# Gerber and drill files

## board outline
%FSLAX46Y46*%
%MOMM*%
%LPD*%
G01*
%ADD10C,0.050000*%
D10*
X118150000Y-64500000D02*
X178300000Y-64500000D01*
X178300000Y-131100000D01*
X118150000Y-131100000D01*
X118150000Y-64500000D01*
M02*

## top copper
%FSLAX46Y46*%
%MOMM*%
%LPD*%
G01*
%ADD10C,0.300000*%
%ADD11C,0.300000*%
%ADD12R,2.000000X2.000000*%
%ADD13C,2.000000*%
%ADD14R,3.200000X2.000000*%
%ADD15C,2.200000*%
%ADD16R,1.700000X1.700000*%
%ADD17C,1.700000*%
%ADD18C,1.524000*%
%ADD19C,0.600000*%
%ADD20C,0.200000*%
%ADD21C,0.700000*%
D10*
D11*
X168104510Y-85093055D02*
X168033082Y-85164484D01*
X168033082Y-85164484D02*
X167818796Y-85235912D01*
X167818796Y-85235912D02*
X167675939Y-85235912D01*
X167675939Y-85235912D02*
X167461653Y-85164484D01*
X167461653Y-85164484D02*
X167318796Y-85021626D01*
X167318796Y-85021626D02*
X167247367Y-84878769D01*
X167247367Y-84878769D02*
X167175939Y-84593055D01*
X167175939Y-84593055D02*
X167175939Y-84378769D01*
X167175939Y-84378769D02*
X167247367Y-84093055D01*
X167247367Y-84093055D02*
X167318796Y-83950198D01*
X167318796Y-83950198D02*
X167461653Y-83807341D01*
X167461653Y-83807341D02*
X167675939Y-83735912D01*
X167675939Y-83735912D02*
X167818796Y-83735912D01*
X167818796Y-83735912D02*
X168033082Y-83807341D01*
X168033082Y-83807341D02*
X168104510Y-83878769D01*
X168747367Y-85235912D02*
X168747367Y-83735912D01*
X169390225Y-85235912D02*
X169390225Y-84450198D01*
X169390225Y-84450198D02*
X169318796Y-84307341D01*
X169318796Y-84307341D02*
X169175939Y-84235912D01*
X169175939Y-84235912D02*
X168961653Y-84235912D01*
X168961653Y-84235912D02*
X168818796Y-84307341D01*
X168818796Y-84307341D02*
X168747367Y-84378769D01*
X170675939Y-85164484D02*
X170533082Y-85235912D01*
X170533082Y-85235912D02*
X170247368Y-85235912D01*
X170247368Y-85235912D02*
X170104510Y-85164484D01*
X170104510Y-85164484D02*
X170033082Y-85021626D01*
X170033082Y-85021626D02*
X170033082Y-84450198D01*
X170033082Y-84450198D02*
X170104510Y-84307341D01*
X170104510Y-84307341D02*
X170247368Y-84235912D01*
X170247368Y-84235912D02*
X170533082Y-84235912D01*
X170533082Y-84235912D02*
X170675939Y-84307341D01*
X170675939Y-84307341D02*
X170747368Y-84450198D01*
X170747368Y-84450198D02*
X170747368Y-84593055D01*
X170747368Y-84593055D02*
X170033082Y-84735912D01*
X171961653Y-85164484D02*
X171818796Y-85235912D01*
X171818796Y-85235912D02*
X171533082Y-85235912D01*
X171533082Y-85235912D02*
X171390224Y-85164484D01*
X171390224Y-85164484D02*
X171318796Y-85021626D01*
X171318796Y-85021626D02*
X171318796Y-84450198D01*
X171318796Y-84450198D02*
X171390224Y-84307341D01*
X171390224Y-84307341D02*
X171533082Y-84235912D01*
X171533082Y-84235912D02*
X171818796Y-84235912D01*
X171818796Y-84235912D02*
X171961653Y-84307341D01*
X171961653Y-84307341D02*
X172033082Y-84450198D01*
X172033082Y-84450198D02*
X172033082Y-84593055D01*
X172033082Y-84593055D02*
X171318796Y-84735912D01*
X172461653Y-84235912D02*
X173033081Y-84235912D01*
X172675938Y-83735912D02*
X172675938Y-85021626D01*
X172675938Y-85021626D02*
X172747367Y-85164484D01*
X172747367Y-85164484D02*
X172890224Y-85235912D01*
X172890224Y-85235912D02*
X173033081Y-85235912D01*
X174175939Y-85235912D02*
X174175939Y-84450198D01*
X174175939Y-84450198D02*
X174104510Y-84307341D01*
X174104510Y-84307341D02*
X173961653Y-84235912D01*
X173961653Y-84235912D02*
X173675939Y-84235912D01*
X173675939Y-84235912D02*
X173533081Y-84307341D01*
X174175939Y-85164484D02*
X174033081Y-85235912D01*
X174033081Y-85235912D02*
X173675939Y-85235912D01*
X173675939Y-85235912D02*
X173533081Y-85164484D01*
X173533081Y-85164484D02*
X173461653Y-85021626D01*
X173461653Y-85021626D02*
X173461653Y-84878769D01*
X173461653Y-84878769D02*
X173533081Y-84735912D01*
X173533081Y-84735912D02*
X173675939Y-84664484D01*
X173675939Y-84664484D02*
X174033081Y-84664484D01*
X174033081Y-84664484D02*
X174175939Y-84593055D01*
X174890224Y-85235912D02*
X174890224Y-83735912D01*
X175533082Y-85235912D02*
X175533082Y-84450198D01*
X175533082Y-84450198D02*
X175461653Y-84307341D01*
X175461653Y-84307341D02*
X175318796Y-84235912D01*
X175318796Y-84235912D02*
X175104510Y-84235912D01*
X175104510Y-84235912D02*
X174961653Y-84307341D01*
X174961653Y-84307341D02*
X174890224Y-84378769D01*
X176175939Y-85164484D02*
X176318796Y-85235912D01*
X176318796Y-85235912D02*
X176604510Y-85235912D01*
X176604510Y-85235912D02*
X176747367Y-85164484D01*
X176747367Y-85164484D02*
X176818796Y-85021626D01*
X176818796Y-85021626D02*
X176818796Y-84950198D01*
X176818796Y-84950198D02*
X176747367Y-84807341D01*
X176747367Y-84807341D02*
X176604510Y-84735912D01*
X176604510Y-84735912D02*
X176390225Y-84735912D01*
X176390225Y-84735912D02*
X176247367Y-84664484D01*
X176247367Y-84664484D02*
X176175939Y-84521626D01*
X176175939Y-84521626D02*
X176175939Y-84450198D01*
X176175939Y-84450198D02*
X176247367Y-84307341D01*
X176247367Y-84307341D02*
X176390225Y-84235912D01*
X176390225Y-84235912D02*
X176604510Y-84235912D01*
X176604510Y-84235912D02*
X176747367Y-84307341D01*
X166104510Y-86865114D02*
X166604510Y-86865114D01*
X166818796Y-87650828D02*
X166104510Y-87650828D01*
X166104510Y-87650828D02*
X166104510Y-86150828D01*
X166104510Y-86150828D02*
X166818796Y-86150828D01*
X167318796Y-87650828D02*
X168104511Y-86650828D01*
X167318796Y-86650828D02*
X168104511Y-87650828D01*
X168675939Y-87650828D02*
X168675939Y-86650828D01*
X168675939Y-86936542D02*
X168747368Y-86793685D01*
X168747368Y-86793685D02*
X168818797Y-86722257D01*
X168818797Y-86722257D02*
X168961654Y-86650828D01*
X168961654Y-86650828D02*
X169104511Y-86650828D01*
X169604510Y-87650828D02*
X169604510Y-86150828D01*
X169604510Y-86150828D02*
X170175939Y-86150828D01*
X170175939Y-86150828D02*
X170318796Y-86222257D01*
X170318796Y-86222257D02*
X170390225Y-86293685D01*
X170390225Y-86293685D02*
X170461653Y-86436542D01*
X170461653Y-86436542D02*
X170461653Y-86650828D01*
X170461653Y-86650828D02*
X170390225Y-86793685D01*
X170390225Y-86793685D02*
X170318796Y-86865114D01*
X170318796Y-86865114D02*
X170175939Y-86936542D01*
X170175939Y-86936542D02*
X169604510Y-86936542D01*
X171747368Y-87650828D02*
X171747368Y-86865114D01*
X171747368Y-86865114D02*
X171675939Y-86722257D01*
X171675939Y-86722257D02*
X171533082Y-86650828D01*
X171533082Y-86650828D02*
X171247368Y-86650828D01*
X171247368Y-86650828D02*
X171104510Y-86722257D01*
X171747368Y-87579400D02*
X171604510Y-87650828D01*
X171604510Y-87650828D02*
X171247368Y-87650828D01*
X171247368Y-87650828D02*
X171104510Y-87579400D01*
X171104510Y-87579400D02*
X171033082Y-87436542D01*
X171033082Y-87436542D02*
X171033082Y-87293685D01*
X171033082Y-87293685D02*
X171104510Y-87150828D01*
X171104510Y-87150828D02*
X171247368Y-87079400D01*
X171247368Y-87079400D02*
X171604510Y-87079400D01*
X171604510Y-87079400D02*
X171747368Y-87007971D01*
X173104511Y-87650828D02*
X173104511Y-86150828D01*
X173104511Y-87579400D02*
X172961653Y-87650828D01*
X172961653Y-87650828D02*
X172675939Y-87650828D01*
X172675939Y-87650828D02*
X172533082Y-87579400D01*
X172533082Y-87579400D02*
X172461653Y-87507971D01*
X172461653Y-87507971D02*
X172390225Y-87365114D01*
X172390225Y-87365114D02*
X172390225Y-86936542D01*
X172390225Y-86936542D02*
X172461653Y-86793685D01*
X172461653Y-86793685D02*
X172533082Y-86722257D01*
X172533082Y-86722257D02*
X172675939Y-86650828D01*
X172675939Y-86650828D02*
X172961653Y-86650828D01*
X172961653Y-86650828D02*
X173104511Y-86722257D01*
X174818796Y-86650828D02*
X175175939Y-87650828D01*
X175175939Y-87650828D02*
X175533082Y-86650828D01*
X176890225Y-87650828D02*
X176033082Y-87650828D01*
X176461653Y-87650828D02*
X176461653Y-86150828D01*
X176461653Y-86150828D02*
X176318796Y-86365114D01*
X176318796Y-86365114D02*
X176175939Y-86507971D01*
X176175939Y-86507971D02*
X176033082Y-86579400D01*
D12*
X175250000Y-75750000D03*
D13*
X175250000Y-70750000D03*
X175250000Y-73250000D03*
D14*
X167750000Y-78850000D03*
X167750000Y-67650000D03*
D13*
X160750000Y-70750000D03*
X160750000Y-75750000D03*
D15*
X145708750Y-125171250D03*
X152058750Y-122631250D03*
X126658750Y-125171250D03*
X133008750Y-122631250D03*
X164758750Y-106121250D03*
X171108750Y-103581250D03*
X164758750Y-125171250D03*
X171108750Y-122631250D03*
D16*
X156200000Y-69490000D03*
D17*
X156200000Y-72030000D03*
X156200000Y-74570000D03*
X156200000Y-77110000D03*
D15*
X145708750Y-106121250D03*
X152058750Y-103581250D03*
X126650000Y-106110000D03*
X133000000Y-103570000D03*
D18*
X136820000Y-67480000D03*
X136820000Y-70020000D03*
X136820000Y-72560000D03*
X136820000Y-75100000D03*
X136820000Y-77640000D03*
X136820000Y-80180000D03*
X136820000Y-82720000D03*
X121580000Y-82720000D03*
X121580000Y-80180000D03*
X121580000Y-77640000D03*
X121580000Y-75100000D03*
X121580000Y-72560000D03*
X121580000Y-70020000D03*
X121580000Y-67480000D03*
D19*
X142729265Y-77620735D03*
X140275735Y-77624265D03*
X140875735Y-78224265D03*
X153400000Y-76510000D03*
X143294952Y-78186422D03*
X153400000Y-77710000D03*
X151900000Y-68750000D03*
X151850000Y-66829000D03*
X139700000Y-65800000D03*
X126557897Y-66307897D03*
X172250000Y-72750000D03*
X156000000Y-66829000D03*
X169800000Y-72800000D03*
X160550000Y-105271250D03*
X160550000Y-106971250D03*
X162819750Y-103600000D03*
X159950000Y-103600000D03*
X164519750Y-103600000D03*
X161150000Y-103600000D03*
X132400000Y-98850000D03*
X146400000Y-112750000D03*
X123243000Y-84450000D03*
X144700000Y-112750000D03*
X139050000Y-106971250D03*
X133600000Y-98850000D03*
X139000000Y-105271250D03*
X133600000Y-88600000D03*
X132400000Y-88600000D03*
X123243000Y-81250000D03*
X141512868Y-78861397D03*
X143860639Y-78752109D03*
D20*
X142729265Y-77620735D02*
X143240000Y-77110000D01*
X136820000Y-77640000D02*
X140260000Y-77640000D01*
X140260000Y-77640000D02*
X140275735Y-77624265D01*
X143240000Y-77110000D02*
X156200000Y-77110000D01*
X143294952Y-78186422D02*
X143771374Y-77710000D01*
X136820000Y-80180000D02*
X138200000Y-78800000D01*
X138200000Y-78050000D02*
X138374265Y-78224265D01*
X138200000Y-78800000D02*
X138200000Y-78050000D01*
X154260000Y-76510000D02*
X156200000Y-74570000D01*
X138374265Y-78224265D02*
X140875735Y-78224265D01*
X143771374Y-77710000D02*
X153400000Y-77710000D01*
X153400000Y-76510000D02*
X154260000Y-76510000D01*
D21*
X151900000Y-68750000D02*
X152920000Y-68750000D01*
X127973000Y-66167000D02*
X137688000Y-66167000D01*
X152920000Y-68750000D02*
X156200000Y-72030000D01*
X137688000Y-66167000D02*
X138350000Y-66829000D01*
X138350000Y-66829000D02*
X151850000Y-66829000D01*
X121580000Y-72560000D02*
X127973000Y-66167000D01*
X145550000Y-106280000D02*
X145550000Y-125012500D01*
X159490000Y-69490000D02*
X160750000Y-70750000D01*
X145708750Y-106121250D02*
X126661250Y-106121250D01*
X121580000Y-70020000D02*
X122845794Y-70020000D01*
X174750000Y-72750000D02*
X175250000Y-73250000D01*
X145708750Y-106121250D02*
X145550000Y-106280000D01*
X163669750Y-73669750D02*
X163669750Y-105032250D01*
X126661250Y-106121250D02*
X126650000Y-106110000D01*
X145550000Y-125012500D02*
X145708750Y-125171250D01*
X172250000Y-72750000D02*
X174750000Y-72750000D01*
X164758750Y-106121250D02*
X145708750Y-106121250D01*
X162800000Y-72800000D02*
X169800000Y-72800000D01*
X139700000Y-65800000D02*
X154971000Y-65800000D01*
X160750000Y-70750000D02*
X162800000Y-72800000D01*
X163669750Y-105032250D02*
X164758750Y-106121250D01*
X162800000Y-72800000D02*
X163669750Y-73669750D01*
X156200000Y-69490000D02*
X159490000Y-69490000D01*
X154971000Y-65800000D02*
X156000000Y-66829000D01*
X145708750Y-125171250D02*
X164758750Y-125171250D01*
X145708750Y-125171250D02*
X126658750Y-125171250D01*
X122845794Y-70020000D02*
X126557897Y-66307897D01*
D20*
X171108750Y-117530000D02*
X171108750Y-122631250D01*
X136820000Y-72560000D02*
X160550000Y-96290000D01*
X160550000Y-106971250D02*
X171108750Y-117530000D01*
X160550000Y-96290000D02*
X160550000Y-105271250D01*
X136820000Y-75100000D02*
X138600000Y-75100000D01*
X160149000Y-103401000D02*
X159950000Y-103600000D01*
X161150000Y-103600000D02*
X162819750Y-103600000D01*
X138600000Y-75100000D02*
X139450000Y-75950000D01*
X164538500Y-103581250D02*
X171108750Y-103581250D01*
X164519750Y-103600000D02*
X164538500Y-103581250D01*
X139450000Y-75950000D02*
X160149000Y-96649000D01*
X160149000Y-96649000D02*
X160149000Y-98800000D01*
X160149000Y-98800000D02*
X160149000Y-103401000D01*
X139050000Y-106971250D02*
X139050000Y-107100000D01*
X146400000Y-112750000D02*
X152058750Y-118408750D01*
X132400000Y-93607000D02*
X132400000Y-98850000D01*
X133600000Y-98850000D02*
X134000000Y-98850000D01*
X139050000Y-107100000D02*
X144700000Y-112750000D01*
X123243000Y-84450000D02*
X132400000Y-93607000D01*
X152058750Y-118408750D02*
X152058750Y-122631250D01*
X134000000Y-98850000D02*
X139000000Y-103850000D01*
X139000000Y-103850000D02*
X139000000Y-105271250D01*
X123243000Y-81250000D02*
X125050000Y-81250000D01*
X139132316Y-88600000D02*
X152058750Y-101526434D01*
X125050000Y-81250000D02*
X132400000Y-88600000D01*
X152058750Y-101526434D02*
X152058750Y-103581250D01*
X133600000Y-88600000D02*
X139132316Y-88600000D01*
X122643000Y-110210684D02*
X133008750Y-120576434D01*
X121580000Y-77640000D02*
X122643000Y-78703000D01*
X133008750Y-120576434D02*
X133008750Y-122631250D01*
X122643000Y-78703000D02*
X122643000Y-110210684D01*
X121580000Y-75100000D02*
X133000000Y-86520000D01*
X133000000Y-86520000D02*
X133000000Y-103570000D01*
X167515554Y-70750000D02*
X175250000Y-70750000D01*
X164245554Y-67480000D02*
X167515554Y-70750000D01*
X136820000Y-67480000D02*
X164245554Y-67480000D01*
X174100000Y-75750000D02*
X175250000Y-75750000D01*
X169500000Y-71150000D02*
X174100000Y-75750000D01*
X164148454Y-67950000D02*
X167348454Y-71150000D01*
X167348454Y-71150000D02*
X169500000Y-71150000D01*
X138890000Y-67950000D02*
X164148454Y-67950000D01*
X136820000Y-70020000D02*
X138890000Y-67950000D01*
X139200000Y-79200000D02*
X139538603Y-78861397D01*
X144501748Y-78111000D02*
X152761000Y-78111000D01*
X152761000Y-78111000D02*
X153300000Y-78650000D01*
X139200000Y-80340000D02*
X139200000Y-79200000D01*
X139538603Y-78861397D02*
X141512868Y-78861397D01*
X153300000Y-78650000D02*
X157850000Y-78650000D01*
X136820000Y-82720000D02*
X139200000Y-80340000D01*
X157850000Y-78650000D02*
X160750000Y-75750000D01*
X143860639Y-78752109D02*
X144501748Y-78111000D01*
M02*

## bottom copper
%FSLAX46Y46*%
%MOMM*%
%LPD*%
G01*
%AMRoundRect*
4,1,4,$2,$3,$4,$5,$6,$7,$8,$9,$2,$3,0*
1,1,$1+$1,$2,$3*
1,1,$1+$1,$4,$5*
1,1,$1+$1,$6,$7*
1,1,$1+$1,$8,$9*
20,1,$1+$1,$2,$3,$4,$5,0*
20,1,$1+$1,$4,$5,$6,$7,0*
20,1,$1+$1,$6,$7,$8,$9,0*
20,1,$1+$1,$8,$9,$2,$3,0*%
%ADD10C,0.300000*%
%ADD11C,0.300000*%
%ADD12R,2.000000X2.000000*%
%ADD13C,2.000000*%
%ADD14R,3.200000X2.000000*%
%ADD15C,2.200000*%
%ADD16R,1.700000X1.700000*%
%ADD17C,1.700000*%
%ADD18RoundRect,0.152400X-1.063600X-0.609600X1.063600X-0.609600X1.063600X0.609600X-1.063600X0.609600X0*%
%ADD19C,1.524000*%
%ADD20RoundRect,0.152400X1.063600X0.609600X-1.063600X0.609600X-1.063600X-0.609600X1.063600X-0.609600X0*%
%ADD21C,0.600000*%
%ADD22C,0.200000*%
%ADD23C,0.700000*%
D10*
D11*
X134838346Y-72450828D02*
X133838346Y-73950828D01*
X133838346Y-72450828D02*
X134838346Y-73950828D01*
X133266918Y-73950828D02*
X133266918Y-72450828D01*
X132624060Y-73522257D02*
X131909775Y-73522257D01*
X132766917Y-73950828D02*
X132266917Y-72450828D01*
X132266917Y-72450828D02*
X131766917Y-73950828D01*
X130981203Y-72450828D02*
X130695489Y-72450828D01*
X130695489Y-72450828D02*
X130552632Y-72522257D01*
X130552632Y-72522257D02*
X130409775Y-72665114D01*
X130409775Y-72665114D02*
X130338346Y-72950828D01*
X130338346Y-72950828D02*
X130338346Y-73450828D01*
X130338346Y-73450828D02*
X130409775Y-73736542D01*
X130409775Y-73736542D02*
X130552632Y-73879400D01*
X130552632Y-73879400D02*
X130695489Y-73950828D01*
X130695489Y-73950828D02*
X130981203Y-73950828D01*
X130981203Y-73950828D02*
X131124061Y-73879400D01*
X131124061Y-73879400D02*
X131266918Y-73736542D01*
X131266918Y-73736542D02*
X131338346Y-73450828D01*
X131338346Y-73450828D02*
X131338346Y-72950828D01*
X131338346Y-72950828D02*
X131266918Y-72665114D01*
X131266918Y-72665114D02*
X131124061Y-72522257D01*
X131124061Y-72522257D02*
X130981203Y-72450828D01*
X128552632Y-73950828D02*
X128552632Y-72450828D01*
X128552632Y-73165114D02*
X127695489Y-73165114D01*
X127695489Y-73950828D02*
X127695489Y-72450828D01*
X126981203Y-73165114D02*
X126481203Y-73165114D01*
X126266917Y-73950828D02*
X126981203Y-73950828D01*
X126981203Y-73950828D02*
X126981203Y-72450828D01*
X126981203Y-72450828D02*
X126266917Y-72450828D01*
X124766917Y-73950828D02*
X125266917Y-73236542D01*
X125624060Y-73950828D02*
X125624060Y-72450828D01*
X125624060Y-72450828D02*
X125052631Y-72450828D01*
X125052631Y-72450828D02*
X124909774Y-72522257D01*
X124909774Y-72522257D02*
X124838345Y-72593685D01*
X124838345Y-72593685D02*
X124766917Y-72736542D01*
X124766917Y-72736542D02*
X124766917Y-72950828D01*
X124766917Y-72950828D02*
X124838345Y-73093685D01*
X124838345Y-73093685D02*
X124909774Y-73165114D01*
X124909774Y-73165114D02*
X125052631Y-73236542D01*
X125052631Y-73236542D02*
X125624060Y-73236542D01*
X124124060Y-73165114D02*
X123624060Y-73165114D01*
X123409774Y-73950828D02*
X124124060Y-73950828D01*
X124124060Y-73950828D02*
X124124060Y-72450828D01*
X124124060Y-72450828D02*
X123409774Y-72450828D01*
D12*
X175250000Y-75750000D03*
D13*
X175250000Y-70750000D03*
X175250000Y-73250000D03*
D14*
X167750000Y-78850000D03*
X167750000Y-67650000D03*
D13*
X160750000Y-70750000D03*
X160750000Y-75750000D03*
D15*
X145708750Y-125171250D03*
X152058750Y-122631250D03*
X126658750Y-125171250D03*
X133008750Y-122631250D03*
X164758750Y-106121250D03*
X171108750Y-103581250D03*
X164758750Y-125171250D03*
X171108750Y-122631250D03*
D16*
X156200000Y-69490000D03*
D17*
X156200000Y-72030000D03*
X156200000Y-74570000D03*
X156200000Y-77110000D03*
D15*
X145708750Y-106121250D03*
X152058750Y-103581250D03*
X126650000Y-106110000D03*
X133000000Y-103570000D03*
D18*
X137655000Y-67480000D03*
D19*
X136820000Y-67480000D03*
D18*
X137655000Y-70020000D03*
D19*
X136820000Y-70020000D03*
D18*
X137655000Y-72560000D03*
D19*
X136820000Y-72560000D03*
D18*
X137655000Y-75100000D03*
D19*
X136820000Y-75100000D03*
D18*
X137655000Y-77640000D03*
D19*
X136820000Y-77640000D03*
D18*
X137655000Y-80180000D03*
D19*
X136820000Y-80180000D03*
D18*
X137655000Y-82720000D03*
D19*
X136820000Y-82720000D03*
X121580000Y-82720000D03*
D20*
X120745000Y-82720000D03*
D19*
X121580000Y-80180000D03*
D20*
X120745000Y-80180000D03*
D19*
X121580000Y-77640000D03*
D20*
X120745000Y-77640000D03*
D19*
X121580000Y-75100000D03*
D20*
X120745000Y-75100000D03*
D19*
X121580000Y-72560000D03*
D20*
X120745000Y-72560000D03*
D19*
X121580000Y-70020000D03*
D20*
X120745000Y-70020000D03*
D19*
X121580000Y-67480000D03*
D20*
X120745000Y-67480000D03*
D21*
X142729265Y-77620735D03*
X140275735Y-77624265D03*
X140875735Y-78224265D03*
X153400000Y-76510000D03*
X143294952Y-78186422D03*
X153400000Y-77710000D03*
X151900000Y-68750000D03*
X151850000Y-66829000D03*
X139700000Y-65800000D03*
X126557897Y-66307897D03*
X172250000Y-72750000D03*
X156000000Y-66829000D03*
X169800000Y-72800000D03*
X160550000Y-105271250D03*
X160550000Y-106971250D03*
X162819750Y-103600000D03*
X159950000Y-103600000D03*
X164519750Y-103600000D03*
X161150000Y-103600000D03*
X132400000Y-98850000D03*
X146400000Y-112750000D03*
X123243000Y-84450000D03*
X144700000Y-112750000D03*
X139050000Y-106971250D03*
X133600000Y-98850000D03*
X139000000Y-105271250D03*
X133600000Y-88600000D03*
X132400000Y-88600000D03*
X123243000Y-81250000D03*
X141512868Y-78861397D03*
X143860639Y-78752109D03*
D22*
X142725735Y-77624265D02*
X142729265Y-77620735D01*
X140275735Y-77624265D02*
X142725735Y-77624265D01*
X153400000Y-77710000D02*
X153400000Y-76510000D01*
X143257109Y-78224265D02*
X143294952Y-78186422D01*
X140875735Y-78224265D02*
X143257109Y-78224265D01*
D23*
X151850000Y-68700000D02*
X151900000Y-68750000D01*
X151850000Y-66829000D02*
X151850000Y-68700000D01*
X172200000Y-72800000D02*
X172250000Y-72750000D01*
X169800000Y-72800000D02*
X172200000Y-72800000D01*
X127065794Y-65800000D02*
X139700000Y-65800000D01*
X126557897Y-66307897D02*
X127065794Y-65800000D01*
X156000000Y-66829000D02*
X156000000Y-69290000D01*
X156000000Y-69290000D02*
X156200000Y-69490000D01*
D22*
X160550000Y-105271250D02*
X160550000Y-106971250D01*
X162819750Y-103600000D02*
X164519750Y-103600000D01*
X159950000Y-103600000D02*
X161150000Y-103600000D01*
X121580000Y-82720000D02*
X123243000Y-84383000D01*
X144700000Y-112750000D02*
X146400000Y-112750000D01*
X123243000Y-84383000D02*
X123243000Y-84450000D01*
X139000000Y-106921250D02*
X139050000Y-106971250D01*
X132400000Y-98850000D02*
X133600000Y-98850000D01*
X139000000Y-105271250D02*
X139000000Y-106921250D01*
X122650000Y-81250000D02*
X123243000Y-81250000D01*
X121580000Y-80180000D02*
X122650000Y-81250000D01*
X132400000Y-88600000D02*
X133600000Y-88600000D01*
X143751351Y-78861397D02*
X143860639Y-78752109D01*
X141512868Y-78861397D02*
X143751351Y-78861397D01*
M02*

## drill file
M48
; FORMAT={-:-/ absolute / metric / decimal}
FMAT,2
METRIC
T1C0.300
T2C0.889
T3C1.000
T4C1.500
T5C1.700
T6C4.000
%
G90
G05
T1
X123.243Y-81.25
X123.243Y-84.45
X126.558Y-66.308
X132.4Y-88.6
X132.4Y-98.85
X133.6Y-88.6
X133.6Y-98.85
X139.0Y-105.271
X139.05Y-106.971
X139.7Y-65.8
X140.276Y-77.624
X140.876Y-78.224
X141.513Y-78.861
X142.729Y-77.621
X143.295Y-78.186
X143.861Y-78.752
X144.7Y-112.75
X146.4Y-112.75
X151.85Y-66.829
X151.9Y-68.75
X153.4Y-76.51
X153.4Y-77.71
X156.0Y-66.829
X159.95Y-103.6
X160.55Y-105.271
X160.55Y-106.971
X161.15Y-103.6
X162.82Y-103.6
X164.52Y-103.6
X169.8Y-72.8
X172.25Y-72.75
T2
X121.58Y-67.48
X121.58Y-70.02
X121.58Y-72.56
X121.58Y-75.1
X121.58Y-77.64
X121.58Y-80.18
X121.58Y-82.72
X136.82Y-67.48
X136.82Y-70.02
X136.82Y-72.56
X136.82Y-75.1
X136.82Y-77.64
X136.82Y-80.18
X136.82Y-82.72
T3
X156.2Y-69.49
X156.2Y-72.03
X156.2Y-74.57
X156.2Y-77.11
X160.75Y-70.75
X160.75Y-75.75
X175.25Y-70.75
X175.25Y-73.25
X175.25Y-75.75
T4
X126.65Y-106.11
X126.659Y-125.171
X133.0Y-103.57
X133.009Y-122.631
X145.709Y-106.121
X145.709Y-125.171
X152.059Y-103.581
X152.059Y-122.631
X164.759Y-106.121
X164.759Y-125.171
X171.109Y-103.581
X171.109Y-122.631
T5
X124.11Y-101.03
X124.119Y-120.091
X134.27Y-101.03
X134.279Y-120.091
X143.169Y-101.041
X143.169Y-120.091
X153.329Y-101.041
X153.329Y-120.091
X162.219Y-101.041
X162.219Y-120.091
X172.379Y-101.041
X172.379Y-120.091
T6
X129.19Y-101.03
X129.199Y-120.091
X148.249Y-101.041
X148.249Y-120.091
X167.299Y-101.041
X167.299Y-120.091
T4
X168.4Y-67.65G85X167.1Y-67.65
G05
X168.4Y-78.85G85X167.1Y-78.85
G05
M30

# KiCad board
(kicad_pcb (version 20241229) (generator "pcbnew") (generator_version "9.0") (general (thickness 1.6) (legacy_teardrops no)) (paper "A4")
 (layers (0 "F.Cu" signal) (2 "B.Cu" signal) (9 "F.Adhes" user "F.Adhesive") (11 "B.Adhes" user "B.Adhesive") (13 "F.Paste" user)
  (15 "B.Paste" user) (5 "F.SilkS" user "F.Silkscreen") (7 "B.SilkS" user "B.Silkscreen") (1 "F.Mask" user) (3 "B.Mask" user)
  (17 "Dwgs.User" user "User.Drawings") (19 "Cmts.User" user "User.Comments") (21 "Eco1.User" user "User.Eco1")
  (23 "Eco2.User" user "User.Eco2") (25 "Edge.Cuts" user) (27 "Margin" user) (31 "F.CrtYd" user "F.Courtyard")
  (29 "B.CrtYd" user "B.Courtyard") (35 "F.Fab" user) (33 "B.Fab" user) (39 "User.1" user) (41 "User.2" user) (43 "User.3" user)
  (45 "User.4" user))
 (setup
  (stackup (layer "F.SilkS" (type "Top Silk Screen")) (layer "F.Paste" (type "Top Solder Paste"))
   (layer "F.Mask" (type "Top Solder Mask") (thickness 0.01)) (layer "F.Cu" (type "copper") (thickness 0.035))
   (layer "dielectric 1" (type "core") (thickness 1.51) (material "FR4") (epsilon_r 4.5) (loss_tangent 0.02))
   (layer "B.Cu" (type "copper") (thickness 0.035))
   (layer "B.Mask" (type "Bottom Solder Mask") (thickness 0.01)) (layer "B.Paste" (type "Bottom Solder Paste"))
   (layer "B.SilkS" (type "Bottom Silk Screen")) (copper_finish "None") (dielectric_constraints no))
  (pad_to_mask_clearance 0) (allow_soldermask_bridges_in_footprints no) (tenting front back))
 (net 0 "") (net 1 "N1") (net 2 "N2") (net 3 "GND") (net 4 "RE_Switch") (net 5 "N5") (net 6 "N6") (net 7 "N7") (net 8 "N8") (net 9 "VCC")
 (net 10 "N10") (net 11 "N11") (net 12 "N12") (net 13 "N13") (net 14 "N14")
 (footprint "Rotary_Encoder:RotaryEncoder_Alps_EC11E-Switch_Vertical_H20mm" (layer "F.Cu") (at 175.25 75.75 180)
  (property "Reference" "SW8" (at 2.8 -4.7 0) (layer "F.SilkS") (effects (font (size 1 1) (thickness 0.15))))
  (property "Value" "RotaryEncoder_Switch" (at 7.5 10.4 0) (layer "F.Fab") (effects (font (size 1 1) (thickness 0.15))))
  (pad "A" thru_hole rect (at 0 0 180) (size 2 2) (drill 1) (layers "*.Cu" "*.Mask") (remove_unused_layers no) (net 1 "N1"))
  (pad "B" thru_hole circle (at 0 5 180) (size 2 2) (drill 1) (layers "*.Cu" "*.Mask") (remove_unused_layers no) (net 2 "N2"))
  (pad "C" thru_hole circle (at 0 2.5 180) (size 2 2) (drill 1) (layers "*.Cu" "*.Mask") (remove_unused_layers no) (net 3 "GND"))
  (pad "MP" thru_hole rect (at 7.5 -3.1 180) (size 3.2 2) (drill oval 2.8 1.5) (layers "*.Cu" "*.Mask") (remove_unused_layers no))
  (pad "MP" thru_hole rect (at 7.5 8.1 180) (size 3.2 2) (drill oval 2.8 1.5) (layers "*.Cu" "*.Mask") (remove_unused_layers no))
  (pad "S1" thru_hole circle (at 14.5 5 180) (size 2 2) (drill 1) (layers "*.Cu" "*.Mask") (remove_unused_layers no) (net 3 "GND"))
  (pad "S2" thru_hole circle (at 14.5 0 180) (size 2 2) (drill 1) (layers "*.Cu" "*.Mask") (remove_unused_layers no) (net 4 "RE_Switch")))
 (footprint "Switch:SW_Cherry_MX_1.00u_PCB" (layer "F.Cu") (at 145.70875 125.17125 180)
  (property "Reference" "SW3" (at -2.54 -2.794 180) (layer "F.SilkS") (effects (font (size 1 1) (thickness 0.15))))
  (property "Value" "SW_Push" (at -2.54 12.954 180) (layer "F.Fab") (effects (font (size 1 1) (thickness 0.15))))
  (pad "" np_thru_hole circle (at -7.62 5.08 180) (size 1.7 1.7) (drill 1.7) (layers "*.Cu" "*.Mask"))
  (pad "" np_thru_hole circle (at -2.54 5.08 180) (size 4 4) (drill 4) (layers "*.Cu" "*.Mask"))
  (pad "" np_thru_hole circle (at 2.54 5.08 180) (size 1.7 1.7) (drill 1.7) (layers "*.Cu" "*.Mask"))
  (pad "1" thru_hole circle (at 0 0 180) (size 2.2 2.2) (drill 1.5) (layers "*.Cu" "*.Mask") (remove_unused_layers no) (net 3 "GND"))
  (pad "2" thru_hole circle (at -6.35 2.54 180) (size 2.2 2.2) (drill 1.5) (layers "*.Cu" "*.Mask") (remove_unused_layers no) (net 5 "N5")))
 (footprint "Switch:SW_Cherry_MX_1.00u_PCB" (layer "F.Cu") (at 126.65875 125.17125 180)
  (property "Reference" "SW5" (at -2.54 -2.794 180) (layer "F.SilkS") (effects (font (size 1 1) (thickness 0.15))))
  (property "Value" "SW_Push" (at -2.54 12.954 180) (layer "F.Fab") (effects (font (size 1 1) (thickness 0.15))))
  (pad "" np_thru_hole circle (at -7.62 5.08 180) (size 1.7 1.7) (drill 1.7) (layers "*.Cu" "*.Mask"))
  (pad "" np_thru_hole circle (at -2.54 5.08 180) (size 4 4) (drill 4) (layers "*.Cu" "*.Mask"))
  (pad "" np_thru_hole circle (at 2.54 5.08 180) (size 1.7 1.7) (drill 1.7) (layers "*.Cu" "*.Mask"))
  (pad "1" thru_hole circle (at 0 0 180) (size 2.2 2.2) (drill 1.5) (layers "*.Cu" "*.Mask") (remove_unused_layers no) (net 3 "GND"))
  (pad "2" thru_hole circle (at -6.35 2.54 180) (size 2.2 2.2) (drill 1.5) (layers "*.Cu" "*.Mask") (remove_unused_layers no) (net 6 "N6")))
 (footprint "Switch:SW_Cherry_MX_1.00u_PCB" (layer "F.Cu") (at 164.75875 106.12125 180)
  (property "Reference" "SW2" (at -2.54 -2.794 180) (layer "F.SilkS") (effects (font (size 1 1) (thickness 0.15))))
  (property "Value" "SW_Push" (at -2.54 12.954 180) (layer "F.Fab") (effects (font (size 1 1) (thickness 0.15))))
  (pad "" np_thru_hole circle (at -7.62 5.08 180) (size 1.7 1.7) (drill 1.7) (layers "*.Cu" "*.Mask"))
  (pad "" np_thru_hole circle (at -2.54 5.08 180) (size 4 4) (drill 4) (layers "*.Cu" "*.Mask"))
  (pad "" np_thru_hole circle (at 2.54 5.08 180) (size 1.7 1.7) (drill 1.7) (layers "*.Cu" "*.Mask"))
  (pad "1" thru_hole circle (at 0 0 180) (size 2.2 2.2) (drill 1.5) (layers "*.Cu" "*.Mask") (remove_unused_layers no) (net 3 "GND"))
  (pad "2" thru_hole circle (at -6.35 2.54 180) (size 2.2 2.2) (drill 1.5) (layers "*.Cu" "*.Mask") (remove_unused_layers no) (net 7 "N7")))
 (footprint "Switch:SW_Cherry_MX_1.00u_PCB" (layer "F.Cu") (at 164.75875 125.17125 180)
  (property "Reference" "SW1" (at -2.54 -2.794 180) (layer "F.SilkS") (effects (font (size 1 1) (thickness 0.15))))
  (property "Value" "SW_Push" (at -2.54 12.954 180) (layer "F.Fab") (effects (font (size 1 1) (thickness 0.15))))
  (pad "" np_thru_hole circle (at -7.62 5.08 180) (size 1.7 1.7) (drill 1.7) (layers "*.Cu" "*.Mask"))
  (pad "" np_thru_hole circle (at -2.54 5.08 180) (size 4 4) (drill 4) (layers "*.Cu" "*.Mask"))
  (pad "" np_thru_hole circle (at 2.54 5.08 180) (size 1.7 1.7) (drill 1.7) (layers "*.Cu" "*.Mask"))
  (pad "1" thru_hole circle (at 0 0 180) (size 2.2 2.2) (drill 1.5) (layers "*.Cu" "*.Mask") (remove_unused_layers no) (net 3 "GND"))
  (pad "2" thru_hole circle (at -6.35 2.54 180) (size 2.2 2.2) (drill 1.5) (layers "*.Cu" "*.Mask") (remove_unused_layers no) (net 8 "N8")))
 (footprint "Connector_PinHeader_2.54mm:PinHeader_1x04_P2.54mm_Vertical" (layer "F.Cu") (at 156.2 69.49)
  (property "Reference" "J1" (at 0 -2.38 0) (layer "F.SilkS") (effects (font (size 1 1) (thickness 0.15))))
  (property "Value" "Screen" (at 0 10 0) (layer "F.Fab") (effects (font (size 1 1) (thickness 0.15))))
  (pad "1" thru_hole rect (at 0 0) (size 1.7 1.7) (drill 1) (layers "*.Cu" "*.Mask") (remove_unused_layers no) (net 3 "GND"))
  (pad "2" thru_hole circle (at 0 2.54) (size 1.7 1.7) (drill 1) (layers "*.Cu" "*.Mask") (remove_unused_layers no) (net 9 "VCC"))
  (pad "3" thru_hole circle (at 0 5.08) (size 1.7 1.7) (drill 1) (layers "*.Cu" "*.Mask") (remove_unused_layers no) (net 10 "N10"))
  (pad "4" thru_hole circle (at 0 7.62) (size 1.7 1.7) (drill 1) (layers "*.Cu" "*.Mask") (remove_unused_layers no) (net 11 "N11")))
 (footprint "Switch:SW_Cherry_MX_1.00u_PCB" (layer "F.Cu") (at 145.70875 106.12125 180)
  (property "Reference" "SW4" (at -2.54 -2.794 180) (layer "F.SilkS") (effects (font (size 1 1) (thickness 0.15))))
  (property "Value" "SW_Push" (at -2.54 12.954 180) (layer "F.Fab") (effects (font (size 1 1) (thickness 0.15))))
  (pad "" np_thru_hole circle (at -7.62 5.08 180) (size 1.7 1.7) (drill 1.7) (layers "*.Cu" "*.Mask"))
  (pad "" np_thru_hole circle (at -2.54 5.08 180) (size 4 4) (drill 4) (layers "*.Cu" "*.Mask"))
  (pad "" np_thru_hole circle (at 2.54 5.08 180) (size 1.7 1.7) (drill 1.7) (layers "*.Cu" "*.Mask"))
  (pad "1" thru_hole circle (at 0 0 180) (size 2.2 2.2) (drill 1.5) (layers "*.Cu" "*.Mask") (remove_unused_layers no) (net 3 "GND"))
  (pad "2" thru_hole circle (at -6.35 2.54 180) (size 2.2 2.2) (drill 1.5) (layers "*.Cu" "*.Mask") (remove_unused_layers no) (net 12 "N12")))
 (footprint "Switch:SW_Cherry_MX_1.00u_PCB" (layer "F.Cu") (at 126.65 106.11 180)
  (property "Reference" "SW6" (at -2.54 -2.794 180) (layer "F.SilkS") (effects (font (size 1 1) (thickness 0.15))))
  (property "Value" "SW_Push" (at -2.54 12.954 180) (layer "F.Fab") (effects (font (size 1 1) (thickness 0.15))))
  (pad "" np_thru_hole circle (at -7.62 5.08 180) (size 1.7 1.7) (drill 1.7) (layers "*.Cu" "*.Mask"))
  (pad "" np_thru_hole circle (at -2.54 5.08 180) (size 4 4) (drill 4) (layers "*.Cu" "*.Mask"))
  (pad "" np_thru_hole circle (at 2.54 5.08 180) (size 1.7 1.7) (drill 1.7) (layers "*.Cu" "*.Mask"))
  (pad "1" thru_hole circle (at 0 0 180) (size 2.2 2.2) (drill 1.5) (layers "*.Cu" "*.Mask") (remove_unused_layers no) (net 3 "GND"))
  (pad "2" thru_hole circle (at -6.35 2.54 180) (size 2.2 2.2) (drill 1.5) (layers "*.Cu" "*.Mask") (remove_unused_layers no) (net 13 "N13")))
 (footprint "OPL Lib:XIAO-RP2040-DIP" (layer "B.Cu") (at 129.2 75.1 180)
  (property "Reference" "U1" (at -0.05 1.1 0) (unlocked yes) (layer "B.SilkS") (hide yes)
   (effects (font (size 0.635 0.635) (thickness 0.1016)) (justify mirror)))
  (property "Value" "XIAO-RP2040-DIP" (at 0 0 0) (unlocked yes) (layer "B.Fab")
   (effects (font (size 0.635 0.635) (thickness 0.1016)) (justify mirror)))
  (pad "1" smd roundrect (at -8.455 7.62) (size 2.432 1.524) (layers "B.Cu" "B.Mask") (roundrect_rratio 0.1) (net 2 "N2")
   (thermal_bridge_angle 45))
  (pad "1" thru_hole circle (at -7.62 7.62) (size 1.524 1.524) (drill 0.889) (layers "*.Cu" "*.Mask") (remove_unused_layers no) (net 2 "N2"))
  (pad "2" smd roundrect (at -8.455 5.08) (size 2.432 1.524) (layers "B.Cu" "B.Mask") (roundrect_rratio 0.1) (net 1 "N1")
   (thermal_bridge_angle 45))
  (pad "2" thru_hole circle (at -7.62 5.08) (size 1.524 1.524) (drill 0.889) (layers "*.Cu" "*.Mask") (remove_unused_layers no) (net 1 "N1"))
  (pad "3" smd roundrect (at -8.455 2.54) (size 2.432 1.524) (layers "B.Cu" "B.Mask") (roundrect_rratio 0.1) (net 8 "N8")
   (thermal_bridge_angle 45))
  (pad "3" thru_hole circle (at -7.62 2.54) (size 1.524 1.524) (drill 0.889) (layers "*.Cu" "*.Mask") (remove_unused_layers no) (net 8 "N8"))
  (pad "4" smd roundrect (at -8.455 0) (size 2.432 1.524) (layers "B.Cu" "B.Mask") (roundrect_rratio 0.1) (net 7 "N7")
   (thermal_bridge_angle 45))
  (pad "4" thru_hole circle (at -7.62 0) (size 1.524 1.524) (drill 0.889) (layers "*.Cu" "*.Mask") (remove_unused_layers no) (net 7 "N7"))
  (pad "5" smd roundrect (at -8.455 -2.54) (size 2.432 1.524) (layers "B.Cu" "B.Mask") (roundrect_rratio 0.1) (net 11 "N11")
   (thermal_bridge_angle 45))
  (pad "5" thru_hole circle (at -7.62 -2.54) (size 1.524 1.524) (drill 0.889) (layers "*.Cu" "*.Mask") (remove_unused_layers no)
   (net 11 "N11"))
  (pad "6" smd roundrect (at -8.455 -5.08) (size 2.432 1.524) (layers "B.Cu" "B.Mask") (roundrect_rratio 0.1) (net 10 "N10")
   (thermal_bridge_angle 45))
  (pad "6" thru_hole circle (at -7.62 -5.08) (size 1.524 1.524) (drill 0.889) (layers "*.Cu" "*.Mask") (remove_unused_layers no)
   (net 10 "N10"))
  (pad "7" smd roundrect (at -8.455 -7.62) (size 2.432 1.524) (layers "B.Cu" "B.Mask") (roundrect_rratio 0.1) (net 4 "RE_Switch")
   (thermal_bridge_angle 45))
  (pad "7" thru_hole circle (at -7.62 -7.62) (size 1.524 1.524) (drill 0.889) (layers "*.Cu" "*.Mask") (remove_unused_layers no)
   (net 4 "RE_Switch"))
  (pad "8" thru_hole circle (at 7.62 -7.62 180) (size 1.524 1.524) (drill 0.889) (layers "*.Cu" "*.Mask") (remove_unused_layers no)
   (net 5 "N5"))
  (pad "8" smd roundrect (at 8.455 -7.62 180) (size 2.432 1.524) (layers "B.Cu" "B.Mask") (roundrect_rratio 0.1) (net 5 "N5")
   (thermal_bridge_angle 45))
  (pad "9" thru_hole circle (at 7.62 -5.08 180) (size 1.524 1.524) (drill 0.889) (layers "*.Cu" "*.Mask") (remove_unused_layers no)
   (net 12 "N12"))
  (pad "9" smd roundrect (at 8.455 -5.08 180) (size 2.432 1.524) (layers "B.Cu" "B.Mask") (roundrect_rratio 0.1) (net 12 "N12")
   (thermal_bridge_angle 45))
  (pad "10" thru_hole circle (at 7.62 -2.54 180) (size 1.524 1.524) (drill 0.889) (layers "*.Cu" "*.Mask") (remove_unused_layers no)
   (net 6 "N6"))
  (pad "10" smd roundrect (at 8.455 -2.54 180) (size 2.432 1.524) (layers "B.Cu" "B.Mask") (roundrect_rratio 0.1) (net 6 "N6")
   (thermal_bridge_angle 45))
  (pad "11" thru_hole circle (at 7.62 0 180) (size 1.524 1.524) (drill 0.889) (layers "*.Cu" "*.Mask") (remove_unused_layers no)
   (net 13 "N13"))
  (pad "11" smd roundrect (at 8.455 0 180) (size 2.432 1.524) (layers "B.Cu" "B.Mask") (roundrect_rratio 0.1) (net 13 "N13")
   (thermal_bridge_angle 45))
  (pad "12" thru_hole circle (at 7.62 2.54 180) (size 1.524 1.524) (drill 0.889) (layers "*.Cu" "*.Mask") (remove_unused_layers no)
   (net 9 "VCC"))
  (pad "12" smd roundrect (at 8.455 2.54 180) (size 2.432 1.524) (layers "B.Cu" "B.Mask") (roundrect_rratio 0.1) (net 9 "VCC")
   (thermal_bridge_angle 45))
  (pad "13" thru_hole circle (at 7.62 5.08 180) (size 1.524 1.524) (drill 0.889) (layers "*.Cu" "*.Mask") (remove_unused_layers no)
   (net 3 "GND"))
  (pad "13" smd roundrect (at 8.455 5.08 180) (size 2.432 1.524) (layers "B.Cu" "B.Mask") (roundrect_rratio 0.1) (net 3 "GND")
   (thermal_bridge_angle 45))
  (pad "14" thru_hole circle (at 7.62 7.62 180) (size 1.524 1.524) (drill 0.889) (layers "*.Cu" "*.Mask") (remove_unused_layers no)
   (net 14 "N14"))
  (pad "14" smd roundrect (at 8.455 7.62 180) (size 2.432 1.524) (layers "B.Cu" "B.Mask") (roundrect_rratio 0.1) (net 14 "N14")
   (thermal_bridge_angle 45)))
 (gr_rect (start 118.15 64.5) (end 178.3 131.1) (stroke (width 0.05) (type default)) (fill no) (layer "Edge.Cuts"))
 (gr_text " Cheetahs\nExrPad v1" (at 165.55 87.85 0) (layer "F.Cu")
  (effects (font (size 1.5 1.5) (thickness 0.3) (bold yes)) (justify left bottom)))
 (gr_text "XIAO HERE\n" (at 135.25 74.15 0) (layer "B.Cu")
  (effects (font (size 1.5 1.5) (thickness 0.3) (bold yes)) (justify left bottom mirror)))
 (segment (start 142.729265 77.620735) (end 143.24 77.11) (width 0.2) (layer "F.Cu") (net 11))
 (segment (start 136.82 77.64) (end 140.26 77.64) (width 0.2) (layer "F.Cu") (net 11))
 (segment (start 140.26 77.64) (end 140.275735 77.624265) (width 0.2) (layer "F.Cu") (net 11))
 (segment (start 143.24 77.11) (end 156.2 77.11) (width 0.2) (layer "F.Cu") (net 11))
 (via (at 142.729265 77.620735) (size 0.6) (drill 0.3) (layers "F.Cu" "B.Cu") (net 11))
 (via (at 140.275735 77.624265) (size 0.6) (drill 0.3) (layers "F.Cu" "B.Cu") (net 11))
 (segment (start 142.725735 77.624265) (end 142.729265 77.620735) (width 0.2) (layer "B.Cu") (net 11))
 (segment (start 140.275735 77.624265) (end 142.725735 77.624265) (width 0.2) (layer "B.Cu") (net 11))
 (segment (start 143.294952 78.186422) (end 143.771374 77.71) (width 0.2) (layer "F.Cu") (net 10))
 (segment (start 136.82 80.18) (end 138.2 78.8) (width 0.2) (layer "F.Cu") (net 10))
 (segment (start 138.2 78.05) (end 138.374265 78.224265) (width 0.2) (layer "F.Cu") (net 10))
 (segment (start 138.2 78.8) (end 138.2 78.05) (width 0.2) (layer "F.Cu") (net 10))
 (segment (start 154.26 76.51) (end 156.2 74.57) (width 0.2) (layer "F.Cu") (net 10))
 (segment (start 138.374265 78.224265) (end 140.875735 78.224265) (width 0.2) (layer "F.Cu") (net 10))
 (segment (start 143.771374 77.71) (end 153.4 77.71) (width 0.2) (layer "F.Cu") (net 10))
 (segment (start 153.4 76.51) (end 154.26 76.51) (width 0.2) (layer "F.Cu") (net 10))
 (via (at 140.875735 78.224265) (size 0.6) (drill 0.3) (layers "F.Cu" "B.Cu") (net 10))
 (via (at 153.4 76.51) (size 0.6) (drill 0.3) (layers "F.Cu" "B.Cu") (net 10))
 (via (at 143.294952 78.186422) (size 0.6) (drill 0.3) (layers "F.Cu" "B.Cu") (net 10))
 (via (at 153.4 77.71) (size 0.6) (drill 0.3) (layers "F.Cu" "B.Cu") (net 10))
 (segment (start 153.4 77.71) (end 153.4 76.51) (width 0.2) (layer "B.Cu") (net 10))
 (segment (start 143.257109 78.224265) (end 143.294952 78.186422) (width 0.2) (layer "B.Cu") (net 10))
 (segment (start 140.875735 78.224265) (end 143.257109 78.224265) (width 0.2) (layer "B.Cu") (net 10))
 (segment (start 151.9 68.75) (end 152.92 68.75) (width 0.7) (layer "F.Cu") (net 9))
 (segment (start 127.973 66.167) (end 137.688 66.167) (width 0.7) (layer "F.Cu") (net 9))
 (segment (start 152.92 68.75) (end 156.2 72.03) (width 0.7) (layer "F.Cu") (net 9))
 (segment (start 137.688 66.167) (end 138.35 66.829) (width 0.7) (layer "F.Cu") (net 9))
 (segment (start 138.35 66.829) (end 151.85 66.829) (width 0.7) (layer "F.Cu") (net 9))
 (segment (start 121.58 72.56) (end 127.973 66.167) (width 0.7) (layer "F.Cu") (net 9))
 (via (at 151.9 68.75) (size 0.6) (drill 0.3) (layers "F.Cu" "B.Cu") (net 9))
 (via (at 151.85 66.829) (size 0.6) (drill 0.3) (layers "F.Cu" "B.Cu") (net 9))
 (segment (start 151.85 68.7) (end 151.9 68.75) (width 0.7) (layer "B.Cu") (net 9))
 (segment (start 151.85 66.829) (end 151.85 68.7) (width 0.7) (layer "B.Cu") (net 9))
 (segment (start 145.55 106.28) (end 145.55 125.0125) (width 0.7) (layer "F.Cu") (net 3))
 (segment (start 159.49 69.49) (end 160.75 70.75) (width 0.7) (layer "F.Cu") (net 3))
 (segment (start 145.70875 106.12125) (end 126.66125 106.12125) (width 0.7) (layer "F.Cu") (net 3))
 (segment (start 121.58 70.02) (end 122.845794 70.02) (width 0.7) (layer "F.Cu") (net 3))
 (segment (start 174.75 72.75) (end 175.25 73.25) (width 0.7) (layer "F.Cu") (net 3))
 (segment (start 145.70875 106.12125) (end 145.55 106.28) (width 0.7) (layer "F.Cu") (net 3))
 (segment (start 163.66975 73.66975) (end 163.66975 105.03225) (width 0.7) (layer "F.Cu") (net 3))
 (segment (start 126.66125 106.12125) (end 126.65 106.11) (width 0.7) (layer "F.Cu") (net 3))
 (segment (start 145.55 125.0125) (end 145.70875 125.17125) (width 0.7) (layer "F.Cu") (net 3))
 (segment (start 172.25 72.75) (end 174.75 72.75) (width 0.7) (layer "F.Cu") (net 3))
 (segment (start 164.75875 106.12125) (end 145.70875 106.12125) (width 0.7) (layer "F.Cu") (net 3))
 (segment (start 162.8 72.8) (end 169.8 72.8) (width 0.7) (layer "F.Cu") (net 3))
 (segment (start 139.7 65.8) (end 154.971 65.8) (width 0.7) (layer "F.Cu") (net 3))
 (segment (start 160.75 70.75) (end 162.8 72.8) (width 0.7) (layer "F.Cu") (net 3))
 (segment (start 163.66975 105.03225) (end 164.75875 106.12125) (width 0.7) (layer "F.Cu") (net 3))
 (segment (start 162.8 72.8) (end 163.66975 73.66975) (width 0.7) (layer "F.Cu") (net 3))
 (segment (start 156.2 69.49) (end 159.49 69.49) (width 0.7) (layer "F.Cu") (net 3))
 (segment (start 154.971 65.8) (end 156 66.829) (width 0.7) (layer "F.Cu") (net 3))
 (segment (start 145.70875 125.17125) (end 164.75875 125.17125) (width 0.7) (layer "F.Cu") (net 3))
 (segment (start 145.70875 125.17125) (end 126.65875 125.17125) (width 0.7) (layer "F.Cu") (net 3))
 (segment (start 122.845794 70.02) (end 126.557897 66.307897) (width 0.7) (layer "F.Cu") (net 3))
 (via (at 139.7 65.8) (size 0.6) (drill 0.3) (layers "F.Cu" "B.Cu") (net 3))
 (via (at 126.557897 66.307897) (size 0.6) (drill 0.3) (layers "F.Cu" "B.Cu") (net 3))
 (via (at 172.25 72.75) (size 0.6) (drill 0.3) (layers "F.Cu" "B.Cu") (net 3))
 (via (at 156 66.829) (size 0.6) (drill 0.3) (layers "F.Cu" "B.Cu") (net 3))
 (via (at 169.8 72.8) (size 0.6) (drill 0.3) (layers "F.Cu" "B.Cu") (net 3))
 (segment (start 172.2 72.8) (end 172.25 72.75) (width 0.7) (layer "B.Cu") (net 3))
 (segment (start 169.8 72.8) (end 172.2 72.8) (width 0.7) (layer "B.Cu") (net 3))
 (segment (start 127.065794 65.8) (end 139.7 65.8) (width 0.7) (layer "B.Cu") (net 3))
 (segment (start 126.557897 66.307897) (end 127.065794 65.8) (width 0.7) (layer "B.Cu") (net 3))
 (segment (start 156 66.829) (end 156 69.29) (width 0.7) (layer "B.Cu") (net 3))
 (segment (start 156 69.29) (end 156.2 69.49) (width 0.7) (layer "B.Cu") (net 3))
 (segment (start 171.10875 117.53) (end 171.10875 122.63125) (width 0.2) (layer "F.Cu") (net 8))
 (segment (start 136.82 72.56) (end 160.55 96.29) (width 0.2) (layer "F.Cu") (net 8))
 (segment (start 160.55 106.97125) (end 171.10875 117.53) (width 0.2) (layer "F.Cu") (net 8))
 (segment (start 160.55 96.29) (end 160.55 105.27125) (width 0.2) (layer "F.Cu") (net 8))
 (via (at 160.55 105.27125) (size 0.6) (drill 0.3) (layers "F.Cu" "B.Cu") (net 8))
 (via (at 160.55 106.97125) (size 0.6) (drill 0.3) (layers "F.Cu" "B.Cu") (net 8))
 (segment (start 160.55 105.27125) (end 160.55 106.97125) (width 0.2) (layer "B.Cu") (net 8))
 (segment (start 136.82 75.1) (end 138.6 75.1) (width 0.2) (layer "F.Cu") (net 7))
 (segment (start 160.149 103.401) (end 159.95 103.6) (width 0.2) (layer "F.Cu") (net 7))
 (segment (start 161.15 103.6) (end 162.81975 103.6) (width 0.2) (layer "F.Cu") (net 7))
 (segment (start 138.6 75.1) (end 139.45 75.95) (width 0.2) (layer "F.Cu") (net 7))
 (segment (start 164.5385 103.58125) (end 171.10875 103.58125) (width 0.2) (layer "F.Cu") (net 7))
 (segment (start 164.51975 103.6) (end 164.5385 103.58125) (width 0.2) (layer "F.Cu") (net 7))
 (segment (start 139.45 75.95) (end 160.149 96.649) (width 0.2) (layer "F.Cu") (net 7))
 (segment (start 160.149 96.649) (end 160.149 98.8) (width 0.2) (layer "F.Cu") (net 7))
 (segment (start 160.149 98.8) (end 160.149 103.401) (width 0.2) (layer "F.Cu") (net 7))
 (via (at 162.81975 103.6) (size 0.6) (drill 0.3) (layers "F.Cu" "B.Cu") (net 7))
 (via (at 159.95 103.6) (size 0.6) (drill 0.3) (layers "F.Cu" "B.Cu") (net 7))
 (via (at 164.51975 103.6) (size 0.6) (drill 0.3) (layers "F.Cu" "B.Cu") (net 7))
 (via (at 161.15 103.6) (size 0.6) (drill 0.3) (layers "F.Cu" "B.Cu") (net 7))
 (segment (start 162.81975 103.6) (end 164.51975 103.6) (width 0.2) (layer "B.Cu") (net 7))
 (segment (start 159.95 103.6) (end 161.15 103.6) (width 0.2) (layer "B.Cu") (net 7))
 (segment (start 139.05 106.97125) (end 139.05 107.1) (width 0.2) (layer "F.Cu") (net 5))
 (segment (start 146.4 112.75) (end 152.05875 118.40875) (width 0.2) (layer "F.Cu") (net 5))
 (segment (start 132.4 93.607) (end 132.4 98.85) (width 0.2) (layer "F.Cu") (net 5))
 (segment (start 133.6 98.85) (end 134 98.85) (width 0.2) (layer "F.Cu") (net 5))
 (segment (start 139.05 107.1) (end 144.7 112.75) (width 0.2) (layer "F.Cu") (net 5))
 (segment (start 123.243 84.45) (end 132.4 93.607) (width 0.2) (layer "F.Cu") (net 5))
 (segment (start 152.05875 118.40875) (end 152.05875 122.63125) (width 0.2) (layer "F.Cu") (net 5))
 (segment (start 134 98.85) (end 139 103.85) (width 0.2) (layer "F.Cu") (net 5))
 (segment (start 139 103.85) (end 139 105.27125) (width 0.2) (layer "F.Cu") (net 5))
 (via (at 132.4 98.85) (size 0.6) (drill 0.3) (layers "F.Cu" "B.Cu") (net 5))
 (via (at 146.4 112.75) (size 0.6) (drill 0.3) (layers "F.Cu" "B.Cu") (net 5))
 (via (at 123.243 84.45) (size 0.6) (drill 0.3) (layers "F.Cu" "B.Cu") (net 5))
 (via (at 144.7 112.75) (size 0.6) (drill 0.3) (layers "F.Cu" "B.Cu") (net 5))
 (via (at 139.05 106.97125) (size 0.6) (drill 0.3) (layers "F.Cu" "B.Cu") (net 5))
 (via (at 133.6 98.85) (size 0.6) (drill 0.3) (layers "F.Cu" "B.Cu") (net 5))
 (via (at 139 105.27125) (size 0.6) (drill 0.3) (layers "F.Cu" "B.Cu") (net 5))
 (segment (start 121.58 82.72) (end 123.243 84.383) (width 0.2) (layer "B.Cu") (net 5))
 (segment (start 144.7 112.75) (end 146.4 112.75) (width 0.2) (layer "B.Cu") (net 5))
 (segment (start 123.243 84.383) (end 123.243 84.45) (width 0.2) (layer "B.Cu") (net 5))
 (segment (start 139 106.92125) (end 139.05 106.97125) (width 0.2) (layer "B.Cu") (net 5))
 (segment (start 132.4 98.85) (end 133.6 98.85) (width 0.2) (layer "B.Cu") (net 5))
 (segment (start 139 105.27125) (end 139 106.92125) (width 0.2) (layer "B.Cu") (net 5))
 (segment (start 123.243 81.25) (end 125.05 81.25) (width 0.2) (layer "F.Cu") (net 12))
 (segment (start 139.132316 88.6) (end 152.05875 101.526434) (width 0.2) (layer "F.Cu") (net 12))
 (segment (start 125.05 81.25) (end 132.4 88.6) (width 0.2) (layer "F.Cu") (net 12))
 (segment (start 152.05875 101.526434) (end 152.05875 103.58125) (width 0.2) (layer "F.Cu") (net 12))
 (segment (start 133.6 88.6) (end 139.132316 88.6) (width 0.2) (layer "F.Cu") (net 12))
 (via (at 133.6 88.6) (size 0.6) (drill 0.3) (layers "F.Cu" "B.Cu") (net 12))
 (via (at 132.4 88.6) (size 0.6) (drill 0.3) (layers "F.Cu" "B.Cu") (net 12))
 (via (at 123.243 81.25) (size 0.6) (drill 0.3) (layers "F.Cu" "B.Cu") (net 12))
 (segment (start 122.65 81.25) (end 123.243 81.25) (width 0.2) (layer "B.Cu") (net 12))
 (segment (start 121.58 80.18) (end 122.65 81.25) (width 0.2) (layer "B.Cu") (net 12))
 (segment (start 132.4 88.6) (end 133.6 88.6) (width 0.2) (layer "B.Cu") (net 12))
 (segment (start 122.643 110.210684) (end 133.00875 120.576434) (width 0.2) (layer "F.Cu") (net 6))
 (segment (start 121.58 77.64) (end 122.643 78.703) (width 0.2) (layer "F.Cu") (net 6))
 (segment (start 133.00875 120.576434) (end 133.00875 122.63125) (width 0.2) (layer "F.Cu") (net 6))
 (segment (start 122.643 78.703) (end 122.643 110.210684) (width 0.2) (layer "F.Cu") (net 6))
 (segment (start 121.58 75.1) (end 133 86.52) (width 0.2) (layer "F.Cu") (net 13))
 (segment (start 133 86.52) (end 133 103.57) (width 0.2) (layer "F.Cu") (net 13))
 (segment (start 167.515554 70.75) (end 175.25 70.75) (width 0.2) (layer "F.Cu") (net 2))
 (segment (start 164.245554 67.48) (end 167.515554 70.75) (width 0.2) (layer "F.Cu") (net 2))
 (segment (start 136.82 67.48) (end 164.245554 67.48) (width 0.2) (layer "F.Cu") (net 2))
 (segment (start 174.1 75.75) (end 175.25 75.75) (width 0.2) (layer "F.Cu") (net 1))
 (segment (start 169.5 71.15) (end 174.1 75.75) (width 0.2) (layer "F.Cu") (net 1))
 (segment (start 164.148454 67.95) (end 167.348454 71.15) (width 0.2) (layer "F.Cu") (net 1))
 (segment (start 167.348454 71.15) (end 169.5 71.15) (width 0.2) (layer "F.Cu") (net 1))
 (segment (start 138.89 67.95) (end 164.148454 67.95) (width 0.2) (layer "F.Cu") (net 1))
 (segment (start 136.82 70.02) (end 138.89 67.95) (width 0.2) (layer "F.Cu") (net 1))
 (segment (start 139.2 79.2) (end 139.538603 78.861397) (width 0.2) (layer "F.Cu") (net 4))
 (segment (start 144.501748 78.111) (end 152.761 78.111) (width 0.2) (layer "F.Cu") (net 4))
 (segment (start 152.761 78.111) (end 153.3 78.65) (width 0.2) (layer "F.Cu") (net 4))
 (segment (start 139.2 80.34) (end 139.2 79.2) (width 0.2) (layer "F.Cu") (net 4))
 (segment (start 139.538603 78.861397) (end 141.512868 78.861397) (width 0.2) (layer "F.Cu") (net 4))
 (segment (start 153.3 78.65) (end 157.85 78.65) (width 0.2) (layer "F.Cu") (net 4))
 (segment (start 136.82 82.72) (end 139.2 80.34) (width 0.2) (layer "F.Cu") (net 4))
 (segment (start 157.85 78.65) (end 160.75 75.75) (width 0.2) (layer "F.Cu") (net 4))
 (segment (start 143.860639 78.752109) (end 144.501748 78.111) (width 0.2) (layer "F.Cu") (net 4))
 (via (at 141.512868 78.861397) (size 0.6) (drill 0.3) (layers "F.Cu" "B.Cu") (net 4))
 (via (at 143.860639 78.752109) (size 0.6) (drill 0.3) (layers "F.Cu" "B.Cu") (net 4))
 (segment (start 143.751351 78.861397) (end 143.860639 78.752109) (width 0.2) (layer "B.Cu") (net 4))
 (segment (start 141.512868 78.861397) (end 143.751351 78.861397) (width 0.2) (layer "B.Cu") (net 4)))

